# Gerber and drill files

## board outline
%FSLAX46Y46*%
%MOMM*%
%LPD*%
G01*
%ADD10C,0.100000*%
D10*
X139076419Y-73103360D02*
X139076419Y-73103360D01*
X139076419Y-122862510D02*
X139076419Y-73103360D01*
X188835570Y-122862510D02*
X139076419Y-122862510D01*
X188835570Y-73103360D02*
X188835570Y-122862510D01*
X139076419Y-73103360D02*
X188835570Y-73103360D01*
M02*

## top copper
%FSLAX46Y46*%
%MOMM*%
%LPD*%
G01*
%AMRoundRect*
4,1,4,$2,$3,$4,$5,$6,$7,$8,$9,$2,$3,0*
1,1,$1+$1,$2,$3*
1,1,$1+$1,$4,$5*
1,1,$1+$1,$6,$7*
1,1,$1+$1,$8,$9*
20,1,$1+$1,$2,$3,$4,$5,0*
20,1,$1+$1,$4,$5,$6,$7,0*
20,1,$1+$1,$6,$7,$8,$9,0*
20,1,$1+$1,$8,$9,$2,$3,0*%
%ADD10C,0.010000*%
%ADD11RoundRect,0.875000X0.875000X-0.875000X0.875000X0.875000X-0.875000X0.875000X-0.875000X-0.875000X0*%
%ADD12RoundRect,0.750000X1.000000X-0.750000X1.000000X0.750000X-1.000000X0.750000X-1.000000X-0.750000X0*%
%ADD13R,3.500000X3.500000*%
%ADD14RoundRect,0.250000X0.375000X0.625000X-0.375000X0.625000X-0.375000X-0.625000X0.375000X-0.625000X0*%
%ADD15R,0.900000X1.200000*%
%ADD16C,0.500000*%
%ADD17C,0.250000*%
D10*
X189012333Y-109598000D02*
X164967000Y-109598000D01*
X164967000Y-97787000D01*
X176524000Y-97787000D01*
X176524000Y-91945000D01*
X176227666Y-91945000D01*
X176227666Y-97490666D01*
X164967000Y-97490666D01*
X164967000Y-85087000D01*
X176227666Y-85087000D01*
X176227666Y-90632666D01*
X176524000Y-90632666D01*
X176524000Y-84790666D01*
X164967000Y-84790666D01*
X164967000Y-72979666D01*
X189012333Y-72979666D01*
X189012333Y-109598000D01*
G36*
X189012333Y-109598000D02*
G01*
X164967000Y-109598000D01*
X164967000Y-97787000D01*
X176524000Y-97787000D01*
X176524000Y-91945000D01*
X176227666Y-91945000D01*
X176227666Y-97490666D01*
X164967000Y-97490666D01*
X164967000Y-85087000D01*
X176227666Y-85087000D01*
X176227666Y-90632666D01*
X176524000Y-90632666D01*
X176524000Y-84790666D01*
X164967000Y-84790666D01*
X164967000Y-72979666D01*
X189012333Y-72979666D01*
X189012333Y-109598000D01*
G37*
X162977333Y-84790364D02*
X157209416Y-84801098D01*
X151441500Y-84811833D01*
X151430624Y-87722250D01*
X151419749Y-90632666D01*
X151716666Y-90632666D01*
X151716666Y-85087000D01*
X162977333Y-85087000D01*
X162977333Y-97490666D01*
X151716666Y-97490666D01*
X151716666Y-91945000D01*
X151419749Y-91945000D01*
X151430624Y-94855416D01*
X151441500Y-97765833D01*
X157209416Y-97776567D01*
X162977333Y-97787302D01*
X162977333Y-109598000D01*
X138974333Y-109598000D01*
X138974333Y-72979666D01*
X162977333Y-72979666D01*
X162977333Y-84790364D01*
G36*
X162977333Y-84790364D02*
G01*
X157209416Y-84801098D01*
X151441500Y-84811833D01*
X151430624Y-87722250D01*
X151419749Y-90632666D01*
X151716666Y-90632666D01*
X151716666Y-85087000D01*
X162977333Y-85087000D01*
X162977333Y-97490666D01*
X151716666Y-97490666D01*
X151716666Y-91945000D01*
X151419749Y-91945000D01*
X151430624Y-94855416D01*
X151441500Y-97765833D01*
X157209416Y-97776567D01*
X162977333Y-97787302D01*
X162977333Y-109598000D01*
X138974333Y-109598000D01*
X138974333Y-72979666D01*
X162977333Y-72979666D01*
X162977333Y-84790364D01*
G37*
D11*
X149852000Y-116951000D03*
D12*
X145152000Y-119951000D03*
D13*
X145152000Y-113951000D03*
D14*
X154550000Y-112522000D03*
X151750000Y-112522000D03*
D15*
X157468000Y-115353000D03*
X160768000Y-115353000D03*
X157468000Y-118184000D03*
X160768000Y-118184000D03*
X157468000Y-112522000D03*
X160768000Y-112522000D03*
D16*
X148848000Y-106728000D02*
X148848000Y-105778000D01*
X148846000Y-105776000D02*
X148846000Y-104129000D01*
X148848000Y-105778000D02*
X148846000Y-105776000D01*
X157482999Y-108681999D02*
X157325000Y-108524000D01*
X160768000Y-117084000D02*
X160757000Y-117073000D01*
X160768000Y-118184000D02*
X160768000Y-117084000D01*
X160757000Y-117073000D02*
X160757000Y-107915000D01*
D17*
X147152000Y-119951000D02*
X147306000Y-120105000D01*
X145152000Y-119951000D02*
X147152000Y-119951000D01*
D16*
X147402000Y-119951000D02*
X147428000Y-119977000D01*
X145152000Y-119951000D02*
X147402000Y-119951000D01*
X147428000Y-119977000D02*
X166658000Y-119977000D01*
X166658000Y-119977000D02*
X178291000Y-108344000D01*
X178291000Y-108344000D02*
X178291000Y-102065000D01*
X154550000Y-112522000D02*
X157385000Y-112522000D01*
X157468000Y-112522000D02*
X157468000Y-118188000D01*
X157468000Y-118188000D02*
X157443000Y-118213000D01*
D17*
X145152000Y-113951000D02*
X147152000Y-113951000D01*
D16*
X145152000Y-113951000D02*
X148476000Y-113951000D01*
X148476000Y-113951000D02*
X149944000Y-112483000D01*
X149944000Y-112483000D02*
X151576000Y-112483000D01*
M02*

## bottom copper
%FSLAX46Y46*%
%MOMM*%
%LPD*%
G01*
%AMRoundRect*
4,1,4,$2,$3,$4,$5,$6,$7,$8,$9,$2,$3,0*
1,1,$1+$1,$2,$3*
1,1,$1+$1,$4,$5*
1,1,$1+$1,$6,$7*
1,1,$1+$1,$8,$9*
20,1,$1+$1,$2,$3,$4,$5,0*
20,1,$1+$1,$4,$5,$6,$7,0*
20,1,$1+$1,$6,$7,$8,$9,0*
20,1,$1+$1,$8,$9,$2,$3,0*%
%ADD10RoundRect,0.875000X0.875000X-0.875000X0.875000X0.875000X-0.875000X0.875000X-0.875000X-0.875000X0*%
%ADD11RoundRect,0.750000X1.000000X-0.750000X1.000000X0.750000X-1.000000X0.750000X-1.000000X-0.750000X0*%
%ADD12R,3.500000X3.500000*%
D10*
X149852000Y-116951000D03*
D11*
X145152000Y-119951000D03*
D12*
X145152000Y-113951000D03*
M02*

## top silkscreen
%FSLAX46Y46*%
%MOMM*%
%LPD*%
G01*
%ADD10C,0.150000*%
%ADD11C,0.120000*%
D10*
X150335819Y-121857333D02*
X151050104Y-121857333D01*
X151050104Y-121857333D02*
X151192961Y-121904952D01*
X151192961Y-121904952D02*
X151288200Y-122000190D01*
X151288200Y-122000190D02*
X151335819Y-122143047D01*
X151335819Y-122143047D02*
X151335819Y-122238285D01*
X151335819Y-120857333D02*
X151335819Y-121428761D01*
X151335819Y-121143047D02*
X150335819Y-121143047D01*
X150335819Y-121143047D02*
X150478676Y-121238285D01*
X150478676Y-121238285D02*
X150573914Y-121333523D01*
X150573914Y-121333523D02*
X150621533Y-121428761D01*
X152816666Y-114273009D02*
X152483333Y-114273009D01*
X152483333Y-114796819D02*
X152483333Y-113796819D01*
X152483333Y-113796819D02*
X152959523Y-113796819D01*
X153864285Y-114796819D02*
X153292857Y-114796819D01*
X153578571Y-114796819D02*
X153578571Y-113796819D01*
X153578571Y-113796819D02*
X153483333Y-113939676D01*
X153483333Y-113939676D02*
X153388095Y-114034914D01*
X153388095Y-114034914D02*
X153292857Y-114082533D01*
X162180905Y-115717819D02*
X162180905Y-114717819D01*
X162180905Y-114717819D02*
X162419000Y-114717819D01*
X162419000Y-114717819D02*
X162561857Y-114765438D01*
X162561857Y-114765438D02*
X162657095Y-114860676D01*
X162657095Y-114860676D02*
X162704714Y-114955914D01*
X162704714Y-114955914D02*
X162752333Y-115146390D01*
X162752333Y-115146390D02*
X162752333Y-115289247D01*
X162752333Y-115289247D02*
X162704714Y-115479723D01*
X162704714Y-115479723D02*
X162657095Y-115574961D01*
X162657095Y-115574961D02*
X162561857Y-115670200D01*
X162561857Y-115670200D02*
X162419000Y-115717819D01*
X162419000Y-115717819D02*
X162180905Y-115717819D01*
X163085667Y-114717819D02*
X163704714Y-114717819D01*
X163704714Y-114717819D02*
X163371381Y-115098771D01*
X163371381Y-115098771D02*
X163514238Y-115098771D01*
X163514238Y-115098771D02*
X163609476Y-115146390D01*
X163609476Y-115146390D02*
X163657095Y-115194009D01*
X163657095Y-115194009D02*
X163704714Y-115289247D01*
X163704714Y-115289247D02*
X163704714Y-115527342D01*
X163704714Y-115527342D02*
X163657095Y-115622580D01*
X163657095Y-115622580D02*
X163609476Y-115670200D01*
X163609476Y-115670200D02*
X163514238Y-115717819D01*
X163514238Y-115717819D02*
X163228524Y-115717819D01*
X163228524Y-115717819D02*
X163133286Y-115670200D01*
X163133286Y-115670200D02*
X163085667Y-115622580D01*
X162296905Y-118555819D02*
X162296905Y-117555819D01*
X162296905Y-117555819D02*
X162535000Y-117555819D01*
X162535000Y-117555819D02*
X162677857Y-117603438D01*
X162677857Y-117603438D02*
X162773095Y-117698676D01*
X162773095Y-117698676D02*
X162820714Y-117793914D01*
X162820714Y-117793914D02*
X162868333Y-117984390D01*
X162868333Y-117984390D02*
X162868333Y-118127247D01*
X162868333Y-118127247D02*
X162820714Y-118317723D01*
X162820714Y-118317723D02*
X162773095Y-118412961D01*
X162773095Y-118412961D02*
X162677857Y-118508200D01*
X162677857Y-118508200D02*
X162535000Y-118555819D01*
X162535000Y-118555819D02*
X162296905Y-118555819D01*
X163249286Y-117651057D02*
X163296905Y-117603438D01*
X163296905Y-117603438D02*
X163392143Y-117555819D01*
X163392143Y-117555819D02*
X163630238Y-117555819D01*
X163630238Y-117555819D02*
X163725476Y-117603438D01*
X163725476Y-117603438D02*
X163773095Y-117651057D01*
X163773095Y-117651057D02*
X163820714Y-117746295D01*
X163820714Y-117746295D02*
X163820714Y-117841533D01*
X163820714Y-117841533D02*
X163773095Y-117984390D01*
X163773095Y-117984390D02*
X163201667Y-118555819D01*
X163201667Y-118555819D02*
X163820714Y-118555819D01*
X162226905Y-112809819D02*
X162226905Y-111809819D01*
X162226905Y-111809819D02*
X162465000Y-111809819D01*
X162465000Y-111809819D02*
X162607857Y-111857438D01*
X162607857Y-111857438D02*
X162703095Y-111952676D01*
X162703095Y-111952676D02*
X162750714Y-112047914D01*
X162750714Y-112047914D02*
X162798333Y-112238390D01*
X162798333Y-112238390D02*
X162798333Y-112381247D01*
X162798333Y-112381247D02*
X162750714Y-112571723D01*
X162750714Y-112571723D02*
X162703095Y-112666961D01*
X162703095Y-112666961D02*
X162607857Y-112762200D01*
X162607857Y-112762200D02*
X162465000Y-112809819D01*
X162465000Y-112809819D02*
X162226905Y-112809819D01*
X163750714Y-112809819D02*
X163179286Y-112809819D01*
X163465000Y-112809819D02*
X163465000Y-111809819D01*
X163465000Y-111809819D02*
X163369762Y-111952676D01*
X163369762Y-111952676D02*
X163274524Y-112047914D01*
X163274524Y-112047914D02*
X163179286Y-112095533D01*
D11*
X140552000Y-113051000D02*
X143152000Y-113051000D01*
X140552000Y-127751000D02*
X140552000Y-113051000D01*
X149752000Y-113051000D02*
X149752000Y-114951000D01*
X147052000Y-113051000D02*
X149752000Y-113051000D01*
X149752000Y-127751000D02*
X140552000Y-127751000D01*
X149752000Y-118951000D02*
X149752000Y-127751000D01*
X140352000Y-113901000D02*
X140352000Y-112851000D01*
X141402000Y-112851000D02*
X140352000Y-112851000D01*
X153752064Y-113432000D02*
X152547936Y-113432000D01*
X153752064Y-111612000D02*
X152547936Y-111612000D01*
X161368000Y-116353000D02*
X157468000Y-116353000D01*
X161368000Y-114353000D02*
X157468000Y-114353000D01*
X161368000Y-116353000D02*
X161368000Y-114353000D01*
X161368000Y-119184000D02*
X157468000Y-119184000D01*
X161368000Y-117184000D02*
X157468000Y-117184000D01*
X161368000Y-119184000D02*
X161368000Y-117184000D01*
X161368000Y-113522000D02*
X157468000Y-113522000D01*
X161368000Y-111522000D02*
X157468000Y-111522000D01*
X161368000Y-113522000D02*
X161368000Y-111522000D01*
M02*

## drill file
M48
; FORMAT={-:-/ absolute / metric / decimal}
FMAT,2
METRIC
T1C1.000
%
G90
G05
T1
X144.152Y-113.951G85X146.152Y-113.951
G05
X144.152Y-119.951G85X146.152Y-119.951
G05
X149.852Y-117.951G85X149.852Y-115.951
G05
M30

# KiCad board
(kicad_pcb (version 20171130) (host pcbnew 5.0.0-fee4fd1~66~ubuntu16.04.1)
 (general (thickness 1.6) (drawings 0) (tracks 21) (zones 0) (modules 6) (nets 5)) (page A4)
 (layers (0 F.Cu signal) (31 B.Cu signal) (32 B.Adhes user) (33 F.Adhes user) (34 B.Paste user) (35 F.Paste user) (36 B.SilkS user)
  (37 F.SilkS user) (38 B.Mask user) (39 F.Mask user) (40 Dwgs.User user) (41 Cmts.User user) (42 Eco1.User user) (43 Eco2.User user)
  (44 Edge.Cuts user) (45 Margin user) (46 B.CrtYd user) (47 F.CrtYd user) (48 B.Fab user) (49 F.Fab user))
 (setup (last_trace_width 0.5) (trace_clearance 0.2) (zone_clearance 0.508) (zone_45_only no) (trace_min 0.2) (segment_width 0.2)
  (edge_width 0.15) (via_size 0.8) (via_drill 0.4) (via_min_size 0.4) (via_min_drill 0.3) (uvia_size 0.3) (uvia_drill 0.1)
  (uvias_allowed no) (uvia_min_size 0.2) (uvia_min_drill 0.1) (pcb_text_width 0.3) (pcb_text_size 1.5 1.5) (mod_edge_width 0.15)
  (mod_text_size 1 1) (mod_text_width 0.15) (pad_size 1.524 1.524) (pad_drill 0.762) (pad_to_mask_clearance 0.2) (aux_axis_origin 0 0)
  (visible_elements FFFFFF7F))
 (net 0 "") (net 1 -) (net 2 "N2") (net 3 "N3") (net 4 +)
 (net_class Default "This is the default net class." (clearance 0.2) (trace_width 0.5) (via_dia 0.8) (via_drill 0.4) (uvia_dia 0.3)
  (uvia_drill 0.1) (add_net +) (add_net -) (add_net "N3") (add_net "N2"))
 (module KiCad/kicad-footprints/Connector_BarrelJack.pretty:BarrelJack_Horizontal (layer F.Cu) (at 145.152 113.951 90)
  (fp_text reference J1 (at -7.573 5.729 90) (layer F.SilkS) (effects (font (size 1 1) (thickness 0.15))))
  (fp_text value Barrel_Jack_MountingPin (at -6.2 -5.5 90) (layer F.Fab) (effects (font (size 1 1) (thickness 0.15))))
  (fp_line (start 0.9 -4.6) (end 0.9 -2) (layer F.SilkS) (width 0.12))
  (fp_line (start -13.8 -4.6) (end 0.9 -4.6) (layer F.SilkS) (width 0.12))
  (fp_line (start 0.9 4.6) (end -1 4.6) (layer F.SilkS) (width 0.12))
  (fp_line (start 0.9 1.9) (end 0.9 4.6) (layer F.SilkS) (width 0.12))
  (fp_line (start -13.8 4.6) (end -13.8 -4.6) (layer F.SilkS) (width 0.12))
  (fp_line (start -5 4.6) (end -13.8 4.6) (layer F.SilkS) (width 0.12))
  (fp_line (start 0.05 -4.8) (end 1.1 -4.8) (layer F.SilkS) (width 0.12))
  (fp_line (start 1.1 -3.75) (end 1.1 -4.8) (layer F.SilkS) (width 0.12))
  (pad 3 thru_hole roundrect (at -3 4.7 90) (size 3.5 3.5) (drill oval 3 1) (layers *.Cu *.Mask) (roundrect_rratio 0.25))
  (pad 2 thru_hole roundrect (at -6 0 90) (size 3 3.5) (drill oval 1 3) (layers *.Cu *.Mask) (roundrect_rratio 0.25) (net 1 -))
  (pad 1 thru_hole rect (at 0 0 90) (size 3.5 3.5) (drill oval 1 3) (layers *.Cu *.Mask) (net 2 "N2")))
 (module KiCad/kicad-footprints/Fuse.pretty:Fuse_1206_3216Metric (layer F.Cu) (at 153.15 112.522 180)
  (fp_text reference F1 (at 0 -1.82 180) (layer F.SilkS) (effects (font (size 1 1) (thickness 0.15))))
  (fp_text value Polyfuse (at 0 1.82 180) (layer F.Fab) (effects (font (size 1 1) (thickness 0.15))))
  (fp_line (start -0.602064 -0.91) (end 0.602064 -0.91) (layer F.SilkS) (width 0.12))
  (fp_line (start -0.602064 0.91) (end 0.602064 0.91) (layer F.SilkS) (width 0.12))
  (pad 1 smd roundrect (at -1.4 0 180) (size 1.25 1.75) (layers F.Cu F.Paste F.Mask) (roundrect_rratio 0.2) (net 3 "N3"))
  (pad 2 smd roundrect (at 1.4 0 180) (size 1.25 1.75) (layers F.Cu F.Paste F.Mask) (roundrect_rratio 0.2) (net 2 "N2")))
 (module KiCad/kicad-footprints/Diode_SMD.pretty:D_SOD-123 (layer F.Cu) (at 159.118 115.353 180)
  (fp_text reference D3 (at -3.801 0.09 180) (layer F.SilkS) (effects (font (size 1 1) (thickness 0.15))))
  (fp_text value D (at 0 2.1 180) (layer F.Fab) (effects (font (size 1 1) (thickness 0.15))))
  (fp_line (start -2.25 -1) (end 1.65 -1) (layer F.SilkS) (width 0.12))
  (fp_line (start -2.25 1) (end 1.65 1) (layer F.SilkS) (width 0.12))
  (fp_line (start -2.25 -1) (end -2.25 1) (layer F.SilkS) (width 0.12))
  (pad 2 smd rect (at 1.65 0 180) (size 0.9 1.2) (layers F.Cu F.Paste F.Mask) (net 3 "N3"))
  (pad 1 smd rect (at -1.65 0 180) (size 0.9 1.2) (layers F.Cu F.Paste F.Mask) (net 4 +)))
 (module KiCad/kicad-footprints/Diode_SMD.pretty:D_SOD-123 (layer F.Cu) (at 159.118 118.184 180)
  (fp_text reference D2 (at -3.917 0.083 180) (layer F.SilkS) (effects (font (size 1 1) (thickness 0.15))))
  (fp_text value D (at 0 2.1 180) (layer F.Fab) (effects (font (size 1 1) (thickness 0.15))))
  (fp_line (start -2.25 -1) (end 1.65 -1) (layer F.SilkS) (width 0.12))
  (fp_line (start -2.25 1) (end 1.65 1) (layer F.SilkS) (width 0.12))
  (fp_line (start -2.25 -1) (end -2.25 1) (layer F.SilkS) (width 0.12))
  (pad 2 smd rect (at 1.65 0 180) (size 0.9 1.2) (layers F.Cu F.Paste F.Mask) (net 3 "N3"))
  (pad 1 smd rect (at -1.65 0 180) (size 0.9 1.2) (layers F.Cu F.Paste F.Mask) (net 4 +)))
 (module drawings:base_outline (layer F.Cu) (at 175.254 80.007)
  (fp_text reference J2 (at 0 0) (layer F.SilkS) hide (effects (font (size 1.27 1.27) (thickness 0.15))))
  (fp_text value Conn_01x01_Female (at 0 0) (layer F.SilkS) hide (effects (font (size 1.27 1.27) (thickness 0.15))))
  (fp_line (start -36.177581 -6.90364) (end -36.177581 -6.90364) (layer Edge.Cuts) (width 0.1))
  (fp_line (start -36.177581 42.85551) (end -36.177581 -6.90364) (layer Edge.Cuts) (width 0.1))
  (fp_line (start 13.58157 42.85551) (end -36.177581 42.85551) (layer Edge.Cuts) (width 0.1))
  (fp_line (start 13.58157 -6.90364) (end 13.58157 42.85551) (layer Edge.Cuts) (width 0.1))
  (fp_line (start -36.177581 -6.90364) (end 13.58157 -6.90364) (layer Edge.Cuts) (width 0.1))
  (fp_poly
   (pts (xy 13.758333 29.591) (xy -10.287 29.591) (xy -10.287 17.78) (xy 1.27 17.78) (xy 1.27 11.938) (xy 0.973666 11.938)
    (xy 0.973666 17.483666) (xy -10.287 17.483666) (xy -10.287 5.08) (xy 0.973666 5.08) (xy 0.973666 10.625666) (xy 1.27 10.625666)
    (xy 1.27 4.783666) (xy -10.287 4.783666) (xy -10.287 -7.027334) (xy 13.758333 -7.027334) (xy 13.758333 29.591))
   (layer F.Cu) (width 0.01))
  (fp_poly
   (pts (xy -12.276667 4.783364) (xy -18.044584 4.794098) (xy -23.8125 4.804833) (xy -23.823376 7.71525) (xy -23.834251 10.625666)
    (xy -23.537334 10.625666) (xy -23.537334 5.08) (xy -12.276667 5.08) (xy -12.276667 17.483666) (xy -23.537334 17.483666)
    (xy -23.537334 11.938) (xy -23.834251 11.938) (xy -23.823376 14.848416) (xy -23.8125 17.758833) (xy -18.044584 17.769567)
    (xy -12.276667 17.780302) (xy -12.276667 29.591) (xy -36.279667 29.591) (xy -36.279667 -7.027334) (xy -12.276667 -7.027334)
    (xy -12.276667 4.783364))
   (layer F.Cu) (width 0.01)))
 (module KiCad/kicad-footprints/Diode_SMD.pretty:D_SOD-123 (layer F.Cu) (at 159.118 112.522 180)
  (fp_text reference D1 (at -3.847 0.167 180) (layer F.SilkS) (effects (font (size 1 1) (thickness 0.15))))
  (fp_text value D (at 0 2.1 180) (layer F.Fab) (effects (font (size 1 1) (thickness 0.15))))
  (fp_line (start -2.25 -1) (end 1.65 -1) (layer F.SilkS) (width 0.12))
  (fp_line (start -2.25 1) (end 1.65 1) (layer F.SilkS) (width 0.12))
  (fp_line (start -2.25 -1) (end -2.25 1) (layer F.SilkS) (width 0.12))
  (pad 2 smd rect (at 1.65 0 180) (size 0.9 1.2) (layers F.Cu F.Paste F.Mask) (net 3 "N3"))
  (pad 1 smd rect (at -1.65 0 180) (size 0.9 1.2) (layers F.Cu F.Paste F.Mask) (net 4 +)))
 (segment (start 148.848 106.728) (end 148.848 105.778) (width 0.5) (layer F.Cu) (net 4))
 (segment (start 148.846 105.776) (end 148.846 104.129) (width 0.5) (layer F.Cu) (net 4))
 (segment (start 148.848 105.778) (end 148.846 105.776) (width 0.5) (layer F.Cu) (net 4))
 (segment (start 157.482999 108.681999) (end 157.325 108.524) (width 0.5) (layer F.Cu) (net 4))
 (segment (start 160.768 117.084) (end 160.757 117.073) (width 0.5) (layer F.Cu) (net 4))
 (segment (start 160.768 118.184) (end 160.768 117.084) (width 0.5) (layer F.Cu) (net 4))
 (segment (start 160.757 117.073) (end 160.757 107.915) (width 0.5) (layer F.Cu) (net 4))
 (segment (start 147.152 119.951) (end 147.306 120.105) (width 0.25) (layer F.Cu) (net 1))
 (segment (start 145.152 119.951) (end 147.152 119.951) (width 0.25) (layer F.Cu) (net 1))
 (segment (start 147.402 119.951) (end 147.428 119.977) (width 0.5) (layer F.Cu) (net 1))
 (segment (start 145.152 119.951) (end 147.402 119.951) (width 0.5) (layer F.Cu) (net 1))
 (segment (start 147.428 119.977) (end 166.658 119.977) (width 0.5) (layer F.Cu) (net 1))
 (segment (start 166.658 119.977) (end 178.291 108.344) (width 0.5) (layer F.Cu) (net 1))
 (segment (start 178.291 108.344) (end 178.291 102.065) (width 0.5) (layer F.Cu) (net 1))
 (segment (start 154.55 112.522) (end 157.385 112.522) (width 0.5) (layer F.Cu) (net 3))
 (segment (start 157.468 112.522) (end 157.468 118.188) (width 0.5) (layer F.Cu) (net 3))
 (segment (start 157.468 118.188) (end 157.443 118.213) (width 0.5) (layer F.Cu) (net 3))
 (segment (start 145.152 113.951) (end 147.152 113.951) (width 0.25) (layer F.Cu) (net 2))
 (segment (start 145.152 113.951) (end 148.476 113.951) (width 0.5) (layer F.Cu) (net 2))
 (segment (start 148.476 113.951) (end 149.944 112.483) (width 0.5) (layer F.Cu) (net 2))
 (segment (start 149.944 112.483) (end 151.576 112.483) (width 0.5) (layer F.Cu) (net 2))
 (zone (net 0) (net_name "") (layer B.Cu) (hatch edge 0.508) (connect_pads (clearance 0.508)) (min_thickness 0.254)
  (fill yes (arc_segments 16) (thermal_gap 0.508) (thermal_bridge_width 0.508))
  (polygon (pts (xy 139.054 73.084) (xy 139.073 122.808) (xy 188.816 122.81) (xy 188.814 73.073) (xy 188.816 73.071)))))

